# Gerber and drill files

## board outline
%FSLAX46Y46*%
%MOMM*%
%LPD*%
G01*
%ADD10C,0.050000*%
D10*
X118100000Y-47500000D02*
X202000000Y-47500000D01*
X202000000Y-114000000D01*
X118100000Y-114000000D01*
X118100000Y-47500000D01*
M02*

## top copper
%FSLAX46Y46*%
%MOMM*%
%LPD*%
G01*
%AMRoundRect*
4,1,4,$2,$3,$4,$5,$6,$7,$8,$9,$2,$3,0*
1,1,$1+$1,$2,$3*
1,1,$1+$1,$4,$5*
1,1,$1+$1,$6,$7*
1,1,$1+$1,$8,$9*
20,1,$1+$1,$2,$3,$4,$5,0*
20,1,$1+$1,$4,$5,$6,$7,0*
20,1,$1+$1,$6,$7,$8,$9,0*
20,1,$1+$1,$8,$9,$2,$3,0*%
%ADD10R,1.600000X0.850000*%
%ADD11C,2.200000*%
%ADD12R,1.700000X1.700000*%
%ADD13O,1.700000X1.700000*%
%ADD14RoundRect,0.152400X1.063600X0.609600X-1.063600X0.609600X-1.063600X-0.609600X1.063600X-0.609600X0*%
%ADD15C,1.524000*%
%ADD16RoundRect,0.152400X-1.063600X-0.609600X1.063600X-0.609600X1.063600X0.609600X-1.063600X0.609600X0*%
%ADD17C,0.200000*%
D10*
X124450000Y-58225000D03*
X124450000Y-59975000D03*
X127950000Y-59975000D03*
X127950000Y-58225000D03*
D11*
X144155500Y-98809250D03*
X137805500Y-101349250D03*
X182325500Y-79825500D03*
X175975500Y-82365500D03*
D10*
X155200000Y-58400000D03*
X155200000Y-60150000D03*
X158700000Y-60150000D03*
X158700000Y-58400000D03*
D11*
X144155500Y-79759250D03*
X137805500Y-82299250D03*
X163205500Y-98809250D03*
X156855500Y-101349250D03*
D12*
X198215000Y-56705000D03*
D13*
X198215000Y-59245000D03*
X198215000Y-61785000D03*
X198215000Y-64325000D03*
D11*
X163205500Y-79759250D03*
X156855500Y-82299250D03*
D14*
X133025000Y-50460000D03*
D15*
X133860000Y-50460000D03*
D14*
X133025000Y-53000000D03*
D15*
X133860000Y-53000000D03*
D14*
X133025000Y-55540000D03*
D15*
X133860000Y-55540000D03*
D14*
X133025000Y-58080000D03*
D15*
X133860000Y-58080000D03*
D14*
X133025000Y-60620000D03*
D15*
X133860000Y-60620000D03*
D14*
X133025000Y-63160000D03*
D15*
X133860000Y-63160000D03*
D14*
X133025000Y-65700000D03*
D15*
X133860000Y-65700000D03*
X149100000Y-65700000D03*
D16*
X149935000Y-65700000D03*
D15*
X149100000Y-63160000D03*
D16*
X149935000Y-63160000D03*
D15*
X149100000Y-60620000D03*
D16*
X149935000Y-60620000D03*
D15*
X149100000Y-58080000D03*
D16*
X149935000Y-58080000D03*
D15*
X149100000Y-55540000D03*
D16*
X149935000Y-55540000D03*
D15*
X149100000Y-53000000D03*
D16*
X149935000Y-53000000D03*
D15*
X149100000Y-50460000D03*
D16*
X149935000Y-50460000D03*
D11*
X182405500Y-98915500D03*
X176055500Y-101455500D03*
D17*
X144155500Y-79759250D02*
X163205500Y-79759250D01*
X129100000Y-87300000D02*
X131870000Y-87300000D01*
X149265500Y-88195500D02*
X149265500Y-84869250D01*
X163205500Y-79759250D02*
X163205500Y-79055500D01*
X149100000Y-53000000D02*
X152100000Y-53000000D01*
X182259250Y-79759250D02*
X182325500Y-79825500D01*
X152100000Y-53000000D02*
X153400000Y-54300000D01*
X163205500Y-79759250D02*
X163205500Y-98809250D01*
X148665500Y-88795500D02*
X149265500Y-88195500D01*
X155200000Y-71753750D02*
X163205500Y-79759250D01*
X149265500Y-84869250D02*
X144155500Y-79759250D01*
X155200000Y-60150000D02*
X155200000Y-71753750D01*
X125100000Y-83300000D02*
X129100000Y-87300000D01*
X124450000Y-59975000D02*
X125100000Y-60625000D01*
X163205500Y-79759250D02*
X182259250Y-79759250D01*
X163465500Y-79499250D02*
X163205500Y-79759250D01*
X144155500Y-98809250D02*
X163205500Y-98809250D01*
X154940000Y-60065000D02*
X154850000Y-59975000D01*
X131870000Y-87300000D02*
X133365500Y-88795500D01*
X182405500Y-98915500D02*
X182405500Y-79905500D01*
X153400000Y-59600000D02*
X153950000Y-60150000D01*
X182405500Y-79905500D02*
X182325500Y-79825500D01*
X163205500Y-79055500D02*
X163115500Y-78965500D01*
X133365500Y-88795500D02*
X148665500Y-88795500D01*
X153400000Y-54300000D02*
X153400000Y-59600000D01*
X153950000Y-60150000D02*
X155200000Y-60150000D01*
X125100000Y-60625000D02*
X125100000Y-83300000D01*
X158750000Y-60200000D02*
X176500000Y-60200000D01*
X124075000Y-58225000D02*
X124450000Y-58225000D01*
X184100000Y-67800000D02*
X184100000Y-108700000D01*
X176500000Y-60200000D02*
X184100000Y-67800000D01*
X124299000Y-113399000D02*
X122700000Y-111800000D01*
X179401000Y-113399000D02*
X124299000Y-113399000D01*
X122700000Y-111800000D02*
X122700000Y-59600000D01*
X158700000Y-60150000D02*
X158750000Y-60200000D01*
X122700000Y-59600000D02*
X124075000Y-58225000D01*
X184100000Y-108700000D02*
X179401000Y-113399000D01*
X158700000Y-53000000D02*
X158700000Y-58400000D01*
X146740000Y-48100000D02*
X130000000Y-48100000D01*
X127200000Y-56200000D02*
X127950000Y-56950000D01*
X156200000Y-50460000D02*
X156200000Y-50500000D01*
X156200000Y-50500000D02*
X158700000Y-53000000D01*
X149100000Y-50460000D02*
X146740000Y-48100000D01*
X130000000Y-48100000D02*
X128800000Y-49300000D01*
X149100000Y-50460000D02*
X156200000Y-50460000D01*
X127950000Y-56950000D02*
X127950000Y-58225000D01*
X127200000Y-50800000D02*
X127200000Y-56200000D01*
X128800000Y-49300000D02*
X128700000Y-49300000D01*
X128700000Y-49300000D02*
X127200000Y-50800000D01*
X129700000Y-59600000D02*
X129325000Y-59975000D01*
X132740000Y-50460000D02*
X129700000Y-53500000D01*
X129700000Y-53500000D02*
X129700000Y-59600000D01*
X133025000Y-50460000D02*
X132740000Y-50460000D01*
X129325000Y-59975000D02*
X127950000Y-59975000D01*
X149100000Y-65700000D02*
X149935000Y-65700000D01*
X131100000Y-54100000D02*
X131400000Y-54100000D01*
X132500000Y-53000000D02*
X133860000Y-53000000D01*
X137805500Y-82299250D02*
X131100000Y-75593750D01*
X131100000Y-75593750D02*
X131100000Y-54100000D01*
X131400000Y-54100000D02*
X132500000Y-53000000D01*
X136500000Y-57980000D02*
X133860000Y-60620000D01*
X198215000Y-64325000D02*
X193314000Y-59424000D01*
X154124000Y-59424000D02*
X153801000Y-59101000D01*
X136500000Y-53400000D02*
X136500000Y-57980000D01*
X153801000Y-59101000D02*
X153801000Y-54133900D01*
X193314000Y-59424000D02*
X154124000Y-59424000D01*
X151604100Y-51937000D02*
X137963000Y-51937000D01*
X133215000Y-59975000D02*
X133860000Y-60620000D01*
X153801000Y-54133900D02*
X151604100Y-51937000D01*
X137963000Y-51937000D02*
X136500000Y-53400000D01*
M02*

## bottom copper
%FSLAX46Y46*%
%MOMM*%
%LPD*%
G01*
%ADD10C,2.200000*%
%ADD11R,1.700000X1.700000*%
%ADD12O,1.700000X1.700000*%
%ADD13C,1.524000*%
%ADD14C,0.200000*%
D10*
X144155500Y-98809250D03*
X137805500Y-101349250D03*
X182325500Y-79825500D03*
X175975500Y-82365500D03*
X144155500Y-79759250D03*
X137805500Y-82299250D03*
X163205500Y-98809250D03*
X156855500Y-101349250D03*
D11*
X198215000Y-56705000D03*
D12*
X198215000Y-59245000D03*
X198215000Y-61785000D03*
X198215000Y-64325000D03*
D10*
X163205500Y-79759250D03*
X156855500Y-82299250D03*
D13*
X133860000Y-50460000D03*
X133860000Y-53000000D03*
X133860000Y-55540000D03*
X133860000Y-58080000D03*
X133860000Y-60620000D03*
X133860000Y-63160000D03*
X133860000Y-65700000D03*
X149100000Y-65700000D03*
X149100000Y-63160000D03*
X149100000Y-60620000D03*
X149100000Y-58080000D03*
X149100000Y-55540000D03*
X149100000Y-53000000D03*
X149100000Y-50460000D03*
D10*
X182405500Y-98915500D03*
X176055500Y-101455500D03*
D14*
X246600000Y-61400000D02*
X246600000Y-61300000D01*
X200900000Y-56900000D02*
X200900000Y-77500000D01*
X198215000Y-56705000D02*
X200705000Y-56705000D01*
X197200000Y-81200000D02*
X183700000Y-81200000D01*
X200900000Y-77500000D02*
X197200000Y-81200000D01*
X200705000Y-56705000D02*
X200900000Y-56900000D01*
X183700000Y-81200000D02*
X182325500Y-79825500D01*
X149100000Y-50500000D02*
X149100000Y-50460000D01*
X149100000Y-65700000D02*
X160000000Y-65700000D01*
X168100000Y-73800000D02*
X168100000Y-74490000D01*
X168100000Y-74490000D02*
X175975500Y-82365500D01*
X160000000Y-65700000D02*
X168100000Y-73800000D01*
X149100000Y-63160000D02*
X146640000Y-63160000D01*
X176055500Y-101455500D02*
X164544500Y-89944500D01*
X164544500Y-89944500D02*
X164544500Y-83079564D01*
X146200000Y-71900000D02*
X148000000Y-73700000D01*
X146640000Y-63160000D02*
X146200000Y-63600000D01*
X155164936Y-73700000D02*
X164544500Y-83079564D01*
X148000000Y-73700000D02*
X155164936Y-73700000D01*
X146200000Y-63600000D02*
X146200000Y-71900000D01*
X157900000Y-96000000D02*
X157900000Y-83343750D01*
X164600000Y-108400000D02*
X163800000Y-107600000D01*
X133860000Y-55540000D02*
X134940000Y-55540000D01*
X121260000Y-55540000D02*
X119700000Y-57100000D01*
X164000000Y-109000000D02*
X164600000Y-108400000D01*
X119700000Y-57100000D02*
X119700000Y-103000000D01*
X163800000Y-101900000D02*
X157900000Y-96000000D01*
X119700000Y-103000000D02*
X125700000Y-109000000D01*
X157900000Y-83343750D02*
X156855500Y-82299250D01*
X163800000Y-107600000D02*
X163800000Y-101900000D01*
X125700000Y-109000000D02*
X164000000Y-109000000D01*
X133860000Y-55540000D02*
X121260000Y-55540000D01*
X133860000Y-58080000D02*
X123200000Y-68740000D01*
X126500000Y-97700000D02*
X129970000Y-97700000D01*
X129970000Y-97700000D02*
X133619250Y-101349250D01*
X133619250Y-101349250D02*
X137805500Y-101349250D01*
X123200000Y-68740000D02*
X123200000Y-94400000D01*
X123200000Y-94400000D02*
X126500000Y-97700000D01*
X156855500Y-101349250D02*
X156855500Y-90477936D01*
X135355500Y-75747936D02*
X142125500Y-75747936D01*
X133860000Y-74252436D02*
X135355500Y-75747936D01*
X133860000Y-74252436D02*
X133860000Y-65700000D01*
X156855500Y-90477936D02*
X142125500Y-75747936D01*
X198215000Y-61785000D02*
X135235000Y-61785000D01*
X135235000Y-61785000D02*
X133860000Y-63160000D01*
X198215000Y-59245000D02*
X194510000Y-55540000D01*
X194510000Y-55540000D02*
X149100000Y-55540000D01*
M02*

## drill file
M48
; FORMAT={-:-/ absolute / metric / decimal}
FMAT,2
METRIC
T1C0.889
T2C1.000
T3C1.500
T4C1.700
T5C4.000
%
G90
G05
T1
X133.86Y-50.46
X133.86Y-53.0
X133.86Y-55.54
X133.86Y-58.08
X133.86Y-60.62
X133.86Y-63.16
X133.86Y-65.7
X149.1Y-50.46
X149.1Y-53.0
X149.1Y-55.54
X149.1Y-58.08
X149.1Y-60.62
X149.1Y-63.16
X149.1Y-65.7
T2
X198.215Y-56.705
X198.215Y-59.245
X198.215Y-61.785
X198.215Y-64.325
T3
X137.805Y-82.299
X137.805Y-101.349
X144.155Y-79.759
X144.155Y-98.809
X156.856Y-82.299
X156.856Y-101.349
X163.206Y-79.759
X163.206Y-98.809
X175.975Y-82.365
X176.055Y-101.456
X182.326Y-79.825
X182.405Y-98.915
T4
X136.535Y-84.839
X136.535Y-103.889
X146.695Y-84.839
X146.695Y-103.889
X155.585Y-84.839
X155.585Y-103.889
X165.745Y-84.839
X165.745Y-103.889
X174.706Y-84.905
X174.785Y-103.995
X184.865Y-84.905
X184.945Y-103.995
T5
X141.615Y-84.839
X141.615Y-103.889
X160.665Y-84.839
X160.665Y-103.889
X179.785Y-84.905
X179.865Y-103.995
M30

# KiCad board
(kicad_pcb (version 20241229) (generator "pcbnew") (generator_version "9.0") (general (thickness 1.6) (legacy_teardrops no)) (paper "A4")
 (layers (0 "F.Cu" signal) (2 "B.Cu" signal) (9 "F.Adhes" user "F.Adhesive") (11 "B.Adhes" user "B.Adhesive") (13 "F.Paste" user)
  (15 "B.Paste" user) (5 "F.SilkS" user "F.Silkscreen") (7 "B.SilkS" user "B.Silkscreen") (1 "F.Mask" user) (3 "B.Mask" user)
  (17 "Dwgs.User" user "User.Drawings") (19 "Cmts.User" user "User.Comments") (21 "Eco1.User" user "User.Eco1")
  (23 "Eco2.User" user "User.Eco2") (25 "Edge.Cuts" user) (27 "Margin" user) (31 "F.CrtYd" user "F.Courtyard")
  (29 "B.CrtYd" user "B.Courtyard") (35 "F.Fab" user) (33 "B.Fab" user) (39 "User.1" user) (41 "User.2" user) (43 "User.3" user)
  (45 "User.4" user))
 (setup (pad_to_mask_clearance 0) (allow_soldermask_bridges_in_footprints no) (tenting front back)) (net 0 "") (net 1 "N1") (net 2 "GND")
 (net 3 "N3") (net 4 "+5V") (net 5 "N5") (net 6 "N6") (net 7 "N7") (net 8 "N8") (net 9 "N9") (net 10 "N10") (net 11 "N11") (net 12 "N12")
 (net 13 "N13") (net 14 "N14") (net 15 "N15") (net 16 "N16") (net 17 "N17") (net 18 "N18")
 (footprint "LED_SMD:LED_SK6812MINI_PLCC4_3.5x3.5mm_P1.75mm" (layer "F.Cu") (at 126.2 59.1)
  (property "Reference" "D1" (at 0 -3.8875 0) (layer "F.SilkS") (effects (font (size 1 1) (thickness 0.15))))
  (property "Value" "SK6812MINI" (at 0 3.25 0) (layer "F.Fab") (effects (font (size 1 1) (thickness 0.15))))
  (pad "1" smd rect (at -1.75 -0.875) (size 1.6 0.85) (layers "F.Cu" "F.Mask" "F.Paste") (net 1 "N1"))
  (pad "2" smd rect (at -1.75 0.875) (size 1.6 0.85) (layers "F.Cu" "F.Mask" "F.Paste") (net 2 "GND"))
  (pad "3" smd rect (at 1.75 0.875) (size 1.6 0.85) (layers "F.Cu" "F.Mask" "F.Paste") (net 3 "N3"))
  (pad "4" smd rect (at 1.75 -0.875) (size 1.6 0.85) (layers "F.Cu" "F.Mask" "F.Paste") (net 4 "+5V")))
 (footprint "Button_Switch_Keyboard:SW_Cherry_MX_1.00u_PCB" (layer "F.Cu") (at 144.1555 98.80925)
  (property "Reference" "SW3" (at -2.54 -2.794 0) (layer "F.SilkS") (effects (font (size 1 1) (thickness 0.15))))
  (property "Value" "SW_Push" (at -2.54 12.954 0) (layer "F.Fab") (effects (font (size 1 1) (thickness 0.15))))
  (pad "" np_thru_hole circle (at -7.62 5.08) (size 1.7 1.7) (drill 1.7) (layers "*.Cu" "*.Mask"))
  (pad "" np_thru_hole circle (at -2.54 5.08) (size 4 4) (drill 4) (layers "*.Cu" "*.Mask"))
  (pad "" np_thru_hole circle (at 2.54 5.08) (size 1.7 1.7) (drill 1.7) (layers "*.Cu" "*.Mask"))
  (pad "1" thru_hole circle (at 0 0) (size 2.2 2.2) (drill 1.5) (layers "*.Cu" "*.Mask") (remove_unused_layers no) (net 2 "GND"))
  (pad "2" thru_hole circle (at -6.35 2.54) (size 2.2 2.2) (drill 1.5) (layers "*.Cu" "*.Mask") (remove_unused_layers no) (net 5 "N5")))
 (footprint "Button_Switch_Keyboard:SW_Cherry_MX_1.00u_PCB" (layer "F.Cu") (at 182.3255 79.8255)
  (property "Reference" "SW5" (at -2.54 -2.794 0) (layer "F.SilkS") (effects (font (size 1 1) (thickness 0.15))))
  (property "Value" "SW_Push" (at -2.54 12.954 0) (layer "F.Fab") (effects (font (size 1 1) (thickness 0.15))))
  (pad "" np_thru_hole circle (at -7.62 5.08) (size 1.7 1.7) (drill 1.7) (layers "*.Cu" "*.Mask"))
  (pad "" np_thru_hole circle (at -2.54 5.08) (size 4 4) (drill 4) (layers "*.Cu" "*.Mask"))
  (pad "" np_thru_hole circle (at 2.54 5.08) (size 1.7 1.7) (drill 1.7) (layers "*.Cu" "*.Mask"))
  (pad "1" thru_hole circle (at 0 0) (size 2.2 2.2) (drill 1.5) (layers "*.Cu" "*.Mask") (remove_unused_layers no) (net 2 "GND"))
  (pad "2" thru_hole circle (at -6.35 2.54) (size 2.2 2.2) (drill 1.5) (layers "*.Cu" "*.Mask") (remove_unused_layers no) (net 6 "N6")))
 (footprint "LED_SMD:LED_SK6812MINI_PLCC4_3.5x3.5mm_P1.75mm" (layer "F.Cu") (at 156.95 59.275)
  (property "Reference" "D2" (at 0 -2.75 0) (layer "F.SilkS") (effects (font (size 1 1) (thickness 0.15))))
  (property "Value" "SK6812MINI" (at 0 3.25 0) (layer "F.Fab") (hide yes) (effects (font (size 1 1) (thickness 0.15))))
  (pad "1" smd rect (at -1.75 -0.875) (size 1.6 0.85) (layers "F.Cu" "F.Mask" "F.Paste") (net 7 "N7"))
  (pad "2" smd rect (at -1.75 0.875) (size 1.6 0.85) (layers "F.Cu" "F.Mask" "F.Paste") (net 2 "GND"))
  (pad "3" smd rect (at 1.75 0.875) (size 1.6 0.85) (layers "F.Cu" "F.Mask" "F.Paste") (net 1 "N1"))
  (pad "4" smd rect (at 1.75 -0.875) (size 1.6 0.85) (layers "F.Cu" "F.Mask" "F.Paste") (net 4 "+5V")))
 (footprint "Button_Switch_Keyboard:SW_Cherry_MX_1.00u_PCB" (layer "F.Cu") (at 144.1555 79.75925)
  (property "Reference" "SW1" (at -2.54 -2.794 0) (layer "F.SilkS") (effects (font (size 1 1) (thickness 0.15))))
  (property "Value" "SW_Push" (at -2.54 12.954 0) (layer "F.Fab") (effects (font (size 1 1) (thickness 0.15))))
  (pad "" np_thru_hole circle (at -7.62 5.08) (size 1.7 1.7) (drill 1.7) (layers "*.Cu" "*.Mask"))
  (pad "" np_thru_hole circle (at -2.54 5.08) (size 4 4) (drill 4) (layers "*.Cu" "*.Mask"))
  (pad "" np_thru_hole circle (at 2.54 5.08) (size 1.7 1.7) (drill 1.7) (layers "*.Cu" "*.Mask"))
  (pad "1" thru_hole circle (at 0 0) (size 2.2 2.2) (drill 1.5) (layers "*.Cu" "*.Mask") (remove_unused_layers no) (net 2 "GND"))
  (pad "2" thru_hole circle (at -6.35 2.54) (size 2.2 2.2) (drill 1.5) (layers "*.Cu" "*.Mask") (remove_unused_layers no) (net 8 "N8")))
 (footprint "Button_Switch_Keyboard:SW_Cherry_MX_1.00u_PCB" (layer "F.Cu") (at 163.2055 98.80925)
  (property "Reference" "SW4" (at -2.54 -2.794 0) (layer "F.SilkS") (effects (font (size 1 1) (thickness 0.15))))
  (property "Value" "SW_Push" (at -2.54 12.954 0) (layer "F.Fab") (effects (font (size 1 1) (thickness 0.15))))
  (pad "" np_thru_hole circle (at -7.62 5.08) (size 1.7 1.7) (drill 1.7) (layers "*.Cu" "*.Mask"))
  (pad "" np_thru_hole circle (at -2.54 5.08) (size 4 4) (drill 4) (layers "*.Cu" "*.Mask"))
  (pad "" np_thru_hole circle (at 2.54 5.08) (size 1.7 1.7) (drill 1.7) (layers "*.Cu" "*.Mask"))
  (pad "1" thru_hole circle (at 0 0) (size 2.2 2.2) (drill 1.5) (layers "*.Cu" "*.Mask") (remove_unused_layers no) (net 2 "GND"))
  (pad "2" thru_hole circle (at -6.35 2.54) (size 2.2 2.2) (drill 1.5) (layers "*.Cu" "*.Mask") (remove_unused_layers no) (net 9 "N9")))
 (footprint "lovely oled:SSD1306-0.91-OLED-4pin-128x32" (layer "F.Cu") (at 161.715 54.515)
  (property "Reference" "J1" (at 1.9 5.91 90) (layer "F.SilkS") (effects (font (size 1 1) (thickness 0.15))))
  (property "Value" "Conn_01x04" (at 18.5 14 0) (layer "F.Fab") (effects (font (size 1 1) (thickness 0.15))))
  (pad "1" thru_hole rect (at 36.5 2.19) (size 1.7 1.7) (drill 1) (layers "*.Cu" "*.Mask") (remove_unused_layers no) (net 2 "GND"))
  (pad "2" thru_hole oval (at 36.5 4.73) (size 1.7 1.7) (drill 1) (layers "*.Cu" "*.Mask") (remove_unused_layers no) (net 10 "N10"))
  (pad "3" thru_hole oval (at 36.5 7.27) (size 1.7 1.7) (drill 1) (layers "*.Cu" "*.Mask") (remove_unused_layers no) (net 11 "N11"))
  (pad "4" thru_hole oval (at 36.5 9.81) (size 1.7 1.7) (drill 1) (layers "*.Cu" "*.Mask") (remove_unused_layers no) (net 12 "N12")))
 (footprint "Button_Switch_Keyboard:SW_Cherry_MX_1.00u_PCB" (layer "F.Cu") (at 163.2055 79.75925)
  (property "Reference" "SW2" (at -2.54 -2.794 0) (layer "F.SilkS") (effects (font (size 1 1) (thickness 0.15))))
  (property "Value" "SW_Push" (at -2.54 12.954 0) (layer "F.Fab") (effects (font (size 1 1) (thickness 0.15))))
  (pad "" np_thru_hole circle (at -7.62 5.08) (size 1.7 1.7) (drill 1.7) (layers "*.Cu" "*.Mask"))
  (pad "" np_thru_hole circle (at -2.54 5.08) (size 4 4) (drill 4) (layers "*.Cu" "*.Mask"))
  (pad "" np_thru_hole circle (at 2.54 5.08) (size 1.7 1.7) (drill 1.7) (layers "*.Cu" "*.Mask"))
  (pad "1" thru_hole circle (at 0 0) (size 2.2 2.2) (drill 1.5) (layers "*.Cu" "*.Mask") (remove_unused_layers no) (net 2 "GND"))
  (pad "2" thru_hole circle (at -6.35 2.54) (size 2.2 2.2) (drill 1.5) (layers "*.Cu" "*.Mask") (remove_unused_layers no) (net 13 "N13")))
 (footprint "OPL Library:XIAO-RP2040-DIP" (layer "F.Cu") (at 141.48 58.08)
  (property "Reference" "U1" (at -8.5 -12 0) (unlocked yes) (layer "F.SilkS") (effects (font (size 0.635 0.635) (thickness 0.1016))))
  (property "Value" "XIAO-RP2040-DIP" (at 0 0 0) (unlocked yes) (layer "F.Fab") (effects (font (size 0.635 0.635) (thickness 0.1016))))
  (pad "1" smd roundrect (at -8.455 -7.62 180) (size 2.432 1.524) (layers "F.Cu" "F.Mask") (roundrect_rratio 0.1) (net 3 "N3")
   (thermal_bridge_angle 45))
  (pad "1" thru_hole circle (at -7.62 -7.62 180) (size 1.524 1.524) (drill 0.889) (layers "*.Cu" "*.Mask") (remove_unused_layers no)
   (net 3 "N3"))
  (pad "2" smd roundrect (at -8.455 -5.08 180) (size 2.432 1.524) (layers "F.Cu" "F.Mask") (roundrect_rratio 0.1) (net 8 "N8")
   (thermal_bridge_angle 45))
  (pad "2" thru_hole circle (at -7.62 -5.08 180) (size 1.524 1.524) (drill 0.889) (layers "*.Cu" "*.Mask") (remove_unused_layers no)
   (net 8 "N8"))
  (pad "3" smd roundrect (at -8.455 -2.54 180) (size 2.432 1.524) (layers "F.Cu" "F.Mask") (roundrect_rratio 0.1) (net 13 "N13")
   (thermal_bridge_angle 45))
  (pad "3" thru_hole circle (at -7.62 -2.54 180) (size 1.524 1.524) (drill 0.889) (layers "*.Cu" "*.Mask") (remove_unused_layers no)
   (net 13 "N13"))
  (pad "4" smd roundrect (at -8.455 0 180) (size 2.432 1.524) (layers "F.Cu" "F.Mask") (roundrect_rratio 0.1) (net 5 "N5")
   (thermal_bridge_angle 45))
  (pad "4" thru_hole circle (at -7.62 0 180) (size 1.524 1.524) (drill 0.889) (layers "*.Cu" "*.Mask") (remove_unused_layers no)
   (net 5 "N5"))
  (pad "5" smd roundrect (at -8.455 2.54 180) (size 2.432 1.524) (layers "F.Cu" "F.Mask") (roundrect_rratio 0.1) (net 12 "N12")
   (thermal_bridge_angle 45))
  (pad "5" thru_hole circle (at -7.62 2.54 180) (size 1.524 1.524) (drill 0.889) (layers "*.Cu" "*.Mask") (remove_unused_layers no)
   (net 12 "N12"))
  (pad "6" smd roundrect (at -8.455 5.08 180) (size 2.432 1.524) (layers "F.Cu" "F.Mask") (roundrect_rratio 0.1) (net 11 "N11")
   (thermal_bridge_angle 45))
  (pad "6" thru_hole circle (at -7.62 5.08 180) (size 1.524 1.524) (drill 0.889) (layers "*.Cu" "*.Mask") (remove_unused_layers no)
   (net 11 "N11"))
  (pad "7" smd roundrect (at -8.455 7.62 180) (size 2.432 1.524) (layers "F.Cu" "F.Mask") (roundrect_rratio 0.1) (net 9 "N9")
   (thermal_bridge_angle 45))
  (pad "7" thru_hole circle (at -7.62 7.62 180) (size 1.524 1.524) (drill 0.889) (layers "*.Cu" "*.Mask") (remove_unused_layers no)
   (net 9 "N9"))
  (pad "8" thru_hole circle (at 7.62 7.62) (size 1.524 1.524) (drill 0.889) (layers "*.Cu" "*.Mask") (remove_unused_layers no) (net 6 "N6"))
  (pad "8" smd roundrect (at 8.455 7.62) (size 2.432 1.524) (layers "F.Cu" "F.Mask") (roundrect_rratio 0.1) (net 6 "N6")
   (thermal_bridge_angle 45))
  (pad "9" thru_hole circle (at 7.62 5.08) (size 1.524 1.524) (drill 0.889) (layers "*.Cu" "*.Mask") (remove_unused_layers no)
   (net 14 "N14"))
  (pad "9" smd roundrect (at 8.455 5.08) (size 2.432 1.524) (layers "F.Cu" "F.Mask") (roundrect_rratio 0.1) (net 14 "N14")
   (thermal_bridge_angle 45))
  (pad "10" thru_hole circle (at 7.62 2.54) (size 1.524 1.524) (drill 0.889) (layers "*.Cu" "*.Mask") (remove_unused_layers no)
   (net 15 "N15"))
  (pad "10" smd roundrect (at 8.455 2.54) (size 2.432 1.524) (layers "F.Cu" "F.Mask") (roundrect_rratio 0.1) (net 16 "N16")
   (thermal_bridge_angle 45))
  (pad "11" thru_hole circle (at 7.62 0) (size 1.524 1.524) (drill 0.889) (layers "*.Cu" "*.Mask") (remove_unused_layers no) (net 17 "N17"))
  (pad "11" smd roundrect (at 8.455 0) (size 2.432 1.524) (layers "F.Cu" "F.Mask") (roundrect_rratio 0.1) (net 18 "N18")
   (thermal_bridge_angle 45))
  (pad "12" thru_hole circle (at 7.62 -2.54) (size 1.524 1.524) (drill 0.889) (layers "*.Cu" "*.Mask") (remove_unused_layers no)
   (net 10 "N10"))
  (pad "12" smd roundrect (at 8.455 -2.54) (size 2.432 1.524) (layers "F.Cu" "F.Mask") (roundrect_rratio 0.1) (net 10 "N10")
   (thermal_bridge_angle 45))
  (pad "13" thru_hole circle (at 7.62 -5.08) (size 1.524 1.524) (drill 0.889) (layers "*.Cu" "*.Mask") (remove_unused_layers no)
   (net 2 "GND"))
  (pad "13" smd roundrect (at 8.455 -5.08) (size 2.432 1.524) (layers "F.Cu" "F.Mask") (roundrect_rratio 0.1) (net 2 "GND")
   (thermal_bridge_angle 45))
  (pad "14" thru_hole circle (at 7.62 -7.62) (size 1.524 1.524) (drill 0.889) (layers "*.Cu" "*.Mask") (remove_unused_layers no)
   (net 4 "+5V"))
  (pad "14" smd roundrect (at 8.455 -7.62) (size 2.432 1.524) (layers "F.Cu" "F.Mask") (roundrect_rratio 0.1) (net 4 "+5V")
   (thermal_bridge_angle 45)))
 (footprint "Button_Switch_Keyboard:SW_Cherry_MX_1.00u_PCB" (layer "F.Cu") (at 182.4055 98.9155)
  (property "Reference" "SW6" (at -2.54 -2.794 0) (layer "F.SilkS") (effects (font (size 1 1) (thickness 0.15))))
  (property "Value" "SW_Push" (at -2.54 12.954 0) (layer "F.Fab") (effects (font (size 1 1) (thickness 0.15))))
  (pad "" np_thru_hole circle (at -7.62 5.08) (size 1.7 1.7) (drill 1.7) (layers "*.Cu" "*.Mask"))
  (pad "" np_thru_hole circle (at -2.54 5.08) (size 4 4) (drill 4) (layers "*.Cu" "*.Mask"))
  (pad "" np_thru_hole circle (at 2.54 5.08) (size 1.7 1.7) (drill 1.7) (layers "*.Cu" "*.Mask"))
  (pad "1" thru_hole circle (at 0 0) (size 2.2 2.2) (drill 1.5) (layers "*.Cu" "*.Mask") (remove_unused_layers no) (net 2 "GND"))
  (pad "2" thru_hole circle (at -6.35 2.54) (size 2.2 2.2) (drill 1.5) (layers "*.Cu" "*.Mask") (remove_unused_layers no) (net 14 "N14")))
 (gr_rect (start 118.1 47.5) (end 202 114) (stroke (width 0.05) (type default)) (fill no) (layer "Edge.Cuts"))
 (segment (start 246.6 61.4) (end 246.6 61.3) (width 0.2) (layer "B.Cu") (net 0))
 (segment (start 144.1555 79.75925) (end 163.2055 79.75925) (width 0.2) (layer "F.Cu") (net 2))
 (segment (start 129.1 87.3) (end 131.87 87.3) (width 0.2) (layer "F.Cu") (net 2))
 (segment (start 149.2655 88.1955) (end 149.2655 84.86925) (width 0.2) (layer "F.Cu") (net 2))
 (segment (start 163.2055 79.75925) (end 163.2055 79.0555) (width 0.2) (layer "F.Cu") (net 2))
 (segment (start 149.1 53) (end 152.1 53) (width 0.2) (layer "F.Cu") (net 2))
 (segment (start 182.25925 79.75925) (end 182.3255 79.8255) (width 0.2) (layer "F.Cu") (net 2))
 (segment (start 152.1 53) (end 153.4 54.3) (width 0.2) (layer "F.Cu") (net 2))
 (segment (start 163.2055 79.75925) (end 163.2055 98.80925) (width 0.2) (layer "F.Cu") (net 2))
 (segment (start 148.6655 88.7955) (end 149.2655 88.1955) (width 0.2) (layer "F.Cu") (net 2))
 (segment (start 155.2 71.75375) (end 163.2055 79.75925) (width 0.2) (layer "F.Cu") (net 2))
 (segment (start 149.2655 84.86925) (end 144.1555 79.75925) (width 0.2) (layer "F.Cu") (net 2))
 (segment (start 155.2 60.15) (end 155.2 71.75375) (width 0.2) (layer "F.Cu") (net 2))
 (segment (start 125.1 83.3) (end 129.1 87.3) (width 0.2) (layer "F.Cu") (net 2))
 (segment (start 124.45 59.975) (end 125.1 60.625) (width 0.2) (layer "F.Cu") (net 2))
 (segment (start 163.2055 79.75925) (end 182.25925 79.75925) (width 0.2) (layer "F.Cu") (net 2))
 (segment (start 163.4655 79.49925) (end 163.2055 79.75925) (width 0.2) (layer "F.Cu") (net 2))
 (segment (start 144.1555 98.80925) (end 163.2055 98.80925) (width 0.2) (layer "F.Cu") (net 2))
 (segment (start 154.94 60.065) (end 154.85 59.975) (width 0.2) (layer "F.Cu") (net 2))
 (segment (start 131.87 87.3) (end 133.3655 88.7955) (width 0.2) (layer "F.Cu") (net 2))
 (segment (start 182.4055 98.9155) (end 182.4055 79.9055) (width 0.2) (layer "F.Cu") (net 2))
 (segment (start 153.4 59.6) (end 153.95 60.15) (width 0.2) (layer "F.Cu") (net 2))
 (segment (start 182.4055 79.9055) (end 182.3255 79.8255) (width 0.2) (layer "F.Cu") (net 2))
 (segment (start 163.2055 79.0555) (end 163.1155 78.9655) (width 0.2) (layer "F.Cu") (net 2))
 (segment (start 133.3655 88.7955) (end 148.6655 88.7955) (width 0.2) (layer "F.Cu") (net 2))
 (segment (start 153.4 54.3) (end 153.4 59.6) (width 0.2) (layer "F.Cu") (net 2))
 (segment (start 153.95 60.15) (end 155.2 60.15) (width 0.2) (layer "F.Cu") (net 2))
 (segment (start 125.1 60.625) (end 125.1 83.3) (width 0.2) (layer "F.Cu") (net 2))
 (segment (start 200.9 56.9) (end 200.9 77.5) (width 0.2) (layer "B.Cu") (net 2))
 (segment (start 198.215 56.705) (end 200.705 56.705) (width 0.2) (layer "B.Cu") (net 2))
 (segment (start 197.2 81.2) (end 183.7 81.2) (width 0.2) (layer "B.Cu") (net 2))
 (segment (start 200.9 77.5) (end 197.2 81.2) (width 0.2) (layer "B.Cu") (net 2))
 (segment (start 200.705 56.705) (end 200.9 56.9) (width 0.2) (layer "B.Cu") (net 2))
 (segment (start 183.7 81.2) (end 182.3255 79.8255) (width 0.2) (layer "B.Cu") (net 2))
 (segment (start 158.75 60.2) (end 176.5 60.2) (width 0.2) (layer "F.Cu") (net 1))
 (segment (start 124.075 58.225) (end 124.45 58.225) (width 0.2) (layer "F.Cu") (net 1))
 (segment (start 184.1 67.8) (end 184.1 108.7) (width 0.2) (layer "F.Cu") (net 1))
 (segment (start 176.5 60.2) (end 184.1 67.8) (width 0.2) (layer "F.Cu") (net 1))
 (segment (start 124.299 113.399) (end 122.7 111.8) (width 0.2) (layer "F.Cu") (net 1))
 (segment (start 179.401 113.399) (end 124.299 113.399) (width 0.2) (layer "F.Cu") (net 1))
 (segment (start 122.7 111.8) (end 122.7 59.6) (width 0.2) (layer "F.Cu") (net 1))
 (segment (start 158.7 60.15) (end 158.75 60.2) (width 0.2) (layer "F.Cu") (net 1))
 (segment (start 122.7 59.6) (end 124.075 58.225) (width 0.2) (layer "F.Cu") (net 1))
 (segment (start 184.1 108.7) (end 179.401 113.399) (width 0.2) (layer "F.Cu") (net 1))
 (segment (start 158.7 53) (end 158.7 58.4) (width 0.2) (layer "F.Cu") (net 4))
 (segment (start 146.74 48.1) (end 130 48.1) (width 0.2) (layer "F.Cu") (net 4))
 (segment (start 127.2 56.2) (end 127.95 56.95) (width 0.2) (layer "F.Cu") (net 4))
 (segment (start 156.2 50.46) (end 156.2 50.5) (width 0.2) (layer "F.Cu") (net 4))
 (segment (start 156.2 50.5) (end 158.7 53) (width 0.2) (layer "F.Cu") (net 4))
 (segment (start 149.1 50.46) (end 146.74 48.1) (width 0.2) (layer "F.Cu") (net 4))
 (segment (start 130 48.1) (end 128.8 49.3) (width 0.2) (layer "F.Cu") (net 4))
 (segment (start 149.1 50.46) (end 156.2 50.46) (width 0.2) (layer "F.Cu") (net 4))
 (segment (start 127.95 56.95) (end 127.95 58.225) (width 0.2) (layer "F.Cu") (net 4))
 (segment (start 127.2 50.8) (end 127.2 56.2) (width 0.2) (layer "F.Cu") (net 4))
 (segment (start 128.8 49.3) (end 128.7 49.3) (width 0.2) (layer "F.Cu") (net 4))
 (segment (start 128.7 49.3) (end 127.2 50.8) (width 0.2) (layer "F.Cu") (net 4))
 (segment (start 149.1 50.5) (end 149.1 50.46) (width 0.2) (layer "B.Cu") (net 4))
 (segment (start 129.7 59.6) (end 129.325 59.975) (width 0.2) (layer "F.Cu") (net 3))
 (segment (start 132.74 50.46) (end 129.7 53.5) (width 0.2) (layer "F.Cu") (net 3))
 (segment (start 129.7 53.5) (end 129.7 59.6) (width 0.2) (layer "F.Cu") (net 3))
 (segment (start 133.025 50.46) (end 132.74 50.46) (width 0.2) (layer "F.Cu") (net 3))
 (segment (start 129.325 59.975) (end 127.95 59.975) (width 0.2) (layer "F.Cu") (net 3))
 (segment (start 149.1 65.7) (end 149.935 65.7) (width 0.2) (layer "F.Cu") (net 6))
 (segment (start 149.1 65.7) (end 160 65.7) (width 0.2) (layer "B.Cu") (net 6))
 (segment (start 168.1 73.8) (end 168.1 74.49) (width 0.2) (layer "B.Cu") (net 6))
 (segment (start 168.1 74.49) (end 175.9755 82.3655) (width 0.2) (layer "B.Cu") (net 6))
 (segment (start 160 65.7) (end 168.1 73.8) (width 0.2) (layer "B.Cu") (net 6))
 (segment (start 149.1 63.16) (end 146.64 63.16) (width 0.2) (layer "B.Cu") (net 14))
 (segment (start 176.0555 101.4555) (end 164.5445 89.9445) (width 0.2) (layer "B.Cu") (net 14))
 (segment (start 164.5445 89.9445) (end 164.5445 83.079564) (width 0.2) (layer "B.Cu") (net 14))
 (segment (start 146.2 71.9) (end 148 73.7) (width 0.2) (layer "B.Cu") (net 14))
 (segment (start 146.64 63.16) (end 146.2 63.6) (width 0.2) (layer "B.Cu") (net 14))
 (segment (start 155.164936 73.7) (end 164.5445 83.079564) (width 0.2) (layer "B.Cu") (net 14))
 (segment (start 148 73.7) (end 155.164936 73.7) (width 0.2) (layer "B.Cu") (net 14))
 (segment (start 146.2 63.6) (end 146.2 71.9) (width 0.2) (layer "B.Cu") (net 14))
 (segment (start 131.1 54.1) (end 131.4 54.1) (width 0.2) (layer "F.Cu") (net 8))
 (segment (start 132.5 53) (end 133.86 53) (width 0.2) (layer "F.Cu") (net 8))
 (segment (start 137.8055 82.29925) (end 131.1 75.59375) (width 0.2) (layer "F.Cu") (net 8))
 (segment (start 131.1 75.59375) (end 131.1 54.1) (width 0.2) (layer "F.Cu") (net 8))
 (segment (start 131.4 54.1) (end 132.5 53) (width 0.2) (layer "F.Cu") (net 8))
 (segment (start 157.9 96) (end 157.9 83.34375) (width 0.2) (layer "B.Cu") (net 13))
 (segment (start 164.6 108.4) (end 163.8 107.6) (width 0.2) (layer "B.Cu") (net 13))
 (segment (start 133.86 55.54) (end 134.94 55.54) (width 0.2) (layer "B.Cu") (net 13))
 (segment (start 121.26 55.54) (end 119.7 57.1) (width 0.2) (layer "B.Cu") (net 13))
 (segment (start 164 109) (end 164.6 108.4) (width 0.2) (layer "B.Cu") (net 13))
 (segment (start 119.7 57.1) (end 119.7 103) (width 0.2) (layer "B.Cu") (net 13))
 (segment (start 163.8 101.9) (end 157.9 96) (width 0.2) (layer "B.Cu") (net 13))
 (segment (start 119.7 103) (end 125.7 109) (width 0.2) (layer "B.Cu") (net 13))
 (segment (start 157.9 83.34375) (end 156.8555 82.29925) (width 0.2) (layer "B.Cu") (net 13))
 (segment (start 163.8 107.6) (end 163.8 101.9) (width 0.2) (layer "B.Cu") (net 13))
 (segment (start 125.7 109) (end 164 109) (width 0.2) (layer "B.Cu") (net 13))
 (segment (start 133.86 55.54) (end 121.26 55.54) (width 0.2) (layer "B.Cu") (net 13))
 (segment (start 133.86 58.08) (end 123.2 68.74) (width 0.2) (layer "B.Cu") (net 5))
 (segment (start 126.5 97.7) (end 129.97 97.7) (width 0.2) (layer "B.Cu") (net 5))
 (segment (start 129.97 97.7) (end 133.61925 101.34925) (width 0.2) (layer "B.Cu") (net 5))
 (segment (start 133.61925 101.34925) (end 137.8055 101.34925) (width 0.2) (layer "B.Cu") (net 5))
 (segment (start 123.2 68.74) (end 123.2 94.4) (width 0.2) (layer "B.Cu") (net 5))
 (segment (start 123.2 94.4) (end 126.5 97.7) (width 0.2) (layer "B.Cu") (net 5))
 (segment (start 156.8555 101.34925) (end 156.8555 90.477936) (width 0.2) (layer "B.Cu") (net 9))
 (segment (start 135.3555 75.747936) (end 142.1255 75.747936) (width 0.2) (layer "B.Cu") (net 9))
 (segment (start 133.86 74.252436) (end 135.3555 75.747936) (width 0.2) (layer "B.Cu") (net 9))
 (segment (start 133.86 74.252436) (end 133.86 65.7) (width 0.2) (layer "B.Cu") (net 9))
 (segment (start 156.8555 90.477936) (end 142.1255 75.747936) (width 0.2) (layer "B.Cu") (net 9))
 (segment (start 198.215 61.785) (end 135.235 61.785) (width 0.2) (layer "B.Cu") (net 11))
 (segment (start 135.235 61.785) (end 133.86 63.16) (width 0.2) (layer "B.Cu") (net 11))
 (segment (start 198.215 59.245) (end 194.51 55.54) (width 0.2) (layer "B.Cu") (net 10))
 (segment (start 194.51 55.54) (end 149.1 55.54) (width 0.2) (layer "B.Cu") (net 10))
 (segment (start 136.5 57.98) (end 133.86 60.62) (width 0.2) (layer "F.Cu") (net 12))
 (segment (start 198.215 64.325) (end 193.314 59.424) (width 0.2) (layer "F.Cu") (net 12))
 (segment (start 154.124 59.424) (end 153.801 59.101) (width 0.2) (layer "F.Cu") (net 12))
 (segment (start 136.5 53.4) (end 136.5 57.98) (width 0.2) (layer "F.Cu") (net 12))
 (segment (start 153.801 59.101) (end 153.801 54.1339) (width 0.2) (layer "F.Cu") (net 12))
 (segment (start 193.314 59.424) (end 154.124 59.424) (width 0.2) (layer "F.Cu") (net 12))
 (segment (start 151.6041 51.937) (end 137.963 51.937) (width 0.2) (layer "F.Cu") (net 12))
 (segment (start 133.215 59.975) (end 133.86 60.62) (width 0.2) (layer "F.Cu") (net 12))
 (segment (start 153.801 54.1339) (end 151.6041 51.937) (width 0.2) (layer "F.Cu") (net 12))
 (segment (start 137.963 51.937) (end 136.5 53.4) (width 0.2) (layer "F.Cu") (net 12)))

